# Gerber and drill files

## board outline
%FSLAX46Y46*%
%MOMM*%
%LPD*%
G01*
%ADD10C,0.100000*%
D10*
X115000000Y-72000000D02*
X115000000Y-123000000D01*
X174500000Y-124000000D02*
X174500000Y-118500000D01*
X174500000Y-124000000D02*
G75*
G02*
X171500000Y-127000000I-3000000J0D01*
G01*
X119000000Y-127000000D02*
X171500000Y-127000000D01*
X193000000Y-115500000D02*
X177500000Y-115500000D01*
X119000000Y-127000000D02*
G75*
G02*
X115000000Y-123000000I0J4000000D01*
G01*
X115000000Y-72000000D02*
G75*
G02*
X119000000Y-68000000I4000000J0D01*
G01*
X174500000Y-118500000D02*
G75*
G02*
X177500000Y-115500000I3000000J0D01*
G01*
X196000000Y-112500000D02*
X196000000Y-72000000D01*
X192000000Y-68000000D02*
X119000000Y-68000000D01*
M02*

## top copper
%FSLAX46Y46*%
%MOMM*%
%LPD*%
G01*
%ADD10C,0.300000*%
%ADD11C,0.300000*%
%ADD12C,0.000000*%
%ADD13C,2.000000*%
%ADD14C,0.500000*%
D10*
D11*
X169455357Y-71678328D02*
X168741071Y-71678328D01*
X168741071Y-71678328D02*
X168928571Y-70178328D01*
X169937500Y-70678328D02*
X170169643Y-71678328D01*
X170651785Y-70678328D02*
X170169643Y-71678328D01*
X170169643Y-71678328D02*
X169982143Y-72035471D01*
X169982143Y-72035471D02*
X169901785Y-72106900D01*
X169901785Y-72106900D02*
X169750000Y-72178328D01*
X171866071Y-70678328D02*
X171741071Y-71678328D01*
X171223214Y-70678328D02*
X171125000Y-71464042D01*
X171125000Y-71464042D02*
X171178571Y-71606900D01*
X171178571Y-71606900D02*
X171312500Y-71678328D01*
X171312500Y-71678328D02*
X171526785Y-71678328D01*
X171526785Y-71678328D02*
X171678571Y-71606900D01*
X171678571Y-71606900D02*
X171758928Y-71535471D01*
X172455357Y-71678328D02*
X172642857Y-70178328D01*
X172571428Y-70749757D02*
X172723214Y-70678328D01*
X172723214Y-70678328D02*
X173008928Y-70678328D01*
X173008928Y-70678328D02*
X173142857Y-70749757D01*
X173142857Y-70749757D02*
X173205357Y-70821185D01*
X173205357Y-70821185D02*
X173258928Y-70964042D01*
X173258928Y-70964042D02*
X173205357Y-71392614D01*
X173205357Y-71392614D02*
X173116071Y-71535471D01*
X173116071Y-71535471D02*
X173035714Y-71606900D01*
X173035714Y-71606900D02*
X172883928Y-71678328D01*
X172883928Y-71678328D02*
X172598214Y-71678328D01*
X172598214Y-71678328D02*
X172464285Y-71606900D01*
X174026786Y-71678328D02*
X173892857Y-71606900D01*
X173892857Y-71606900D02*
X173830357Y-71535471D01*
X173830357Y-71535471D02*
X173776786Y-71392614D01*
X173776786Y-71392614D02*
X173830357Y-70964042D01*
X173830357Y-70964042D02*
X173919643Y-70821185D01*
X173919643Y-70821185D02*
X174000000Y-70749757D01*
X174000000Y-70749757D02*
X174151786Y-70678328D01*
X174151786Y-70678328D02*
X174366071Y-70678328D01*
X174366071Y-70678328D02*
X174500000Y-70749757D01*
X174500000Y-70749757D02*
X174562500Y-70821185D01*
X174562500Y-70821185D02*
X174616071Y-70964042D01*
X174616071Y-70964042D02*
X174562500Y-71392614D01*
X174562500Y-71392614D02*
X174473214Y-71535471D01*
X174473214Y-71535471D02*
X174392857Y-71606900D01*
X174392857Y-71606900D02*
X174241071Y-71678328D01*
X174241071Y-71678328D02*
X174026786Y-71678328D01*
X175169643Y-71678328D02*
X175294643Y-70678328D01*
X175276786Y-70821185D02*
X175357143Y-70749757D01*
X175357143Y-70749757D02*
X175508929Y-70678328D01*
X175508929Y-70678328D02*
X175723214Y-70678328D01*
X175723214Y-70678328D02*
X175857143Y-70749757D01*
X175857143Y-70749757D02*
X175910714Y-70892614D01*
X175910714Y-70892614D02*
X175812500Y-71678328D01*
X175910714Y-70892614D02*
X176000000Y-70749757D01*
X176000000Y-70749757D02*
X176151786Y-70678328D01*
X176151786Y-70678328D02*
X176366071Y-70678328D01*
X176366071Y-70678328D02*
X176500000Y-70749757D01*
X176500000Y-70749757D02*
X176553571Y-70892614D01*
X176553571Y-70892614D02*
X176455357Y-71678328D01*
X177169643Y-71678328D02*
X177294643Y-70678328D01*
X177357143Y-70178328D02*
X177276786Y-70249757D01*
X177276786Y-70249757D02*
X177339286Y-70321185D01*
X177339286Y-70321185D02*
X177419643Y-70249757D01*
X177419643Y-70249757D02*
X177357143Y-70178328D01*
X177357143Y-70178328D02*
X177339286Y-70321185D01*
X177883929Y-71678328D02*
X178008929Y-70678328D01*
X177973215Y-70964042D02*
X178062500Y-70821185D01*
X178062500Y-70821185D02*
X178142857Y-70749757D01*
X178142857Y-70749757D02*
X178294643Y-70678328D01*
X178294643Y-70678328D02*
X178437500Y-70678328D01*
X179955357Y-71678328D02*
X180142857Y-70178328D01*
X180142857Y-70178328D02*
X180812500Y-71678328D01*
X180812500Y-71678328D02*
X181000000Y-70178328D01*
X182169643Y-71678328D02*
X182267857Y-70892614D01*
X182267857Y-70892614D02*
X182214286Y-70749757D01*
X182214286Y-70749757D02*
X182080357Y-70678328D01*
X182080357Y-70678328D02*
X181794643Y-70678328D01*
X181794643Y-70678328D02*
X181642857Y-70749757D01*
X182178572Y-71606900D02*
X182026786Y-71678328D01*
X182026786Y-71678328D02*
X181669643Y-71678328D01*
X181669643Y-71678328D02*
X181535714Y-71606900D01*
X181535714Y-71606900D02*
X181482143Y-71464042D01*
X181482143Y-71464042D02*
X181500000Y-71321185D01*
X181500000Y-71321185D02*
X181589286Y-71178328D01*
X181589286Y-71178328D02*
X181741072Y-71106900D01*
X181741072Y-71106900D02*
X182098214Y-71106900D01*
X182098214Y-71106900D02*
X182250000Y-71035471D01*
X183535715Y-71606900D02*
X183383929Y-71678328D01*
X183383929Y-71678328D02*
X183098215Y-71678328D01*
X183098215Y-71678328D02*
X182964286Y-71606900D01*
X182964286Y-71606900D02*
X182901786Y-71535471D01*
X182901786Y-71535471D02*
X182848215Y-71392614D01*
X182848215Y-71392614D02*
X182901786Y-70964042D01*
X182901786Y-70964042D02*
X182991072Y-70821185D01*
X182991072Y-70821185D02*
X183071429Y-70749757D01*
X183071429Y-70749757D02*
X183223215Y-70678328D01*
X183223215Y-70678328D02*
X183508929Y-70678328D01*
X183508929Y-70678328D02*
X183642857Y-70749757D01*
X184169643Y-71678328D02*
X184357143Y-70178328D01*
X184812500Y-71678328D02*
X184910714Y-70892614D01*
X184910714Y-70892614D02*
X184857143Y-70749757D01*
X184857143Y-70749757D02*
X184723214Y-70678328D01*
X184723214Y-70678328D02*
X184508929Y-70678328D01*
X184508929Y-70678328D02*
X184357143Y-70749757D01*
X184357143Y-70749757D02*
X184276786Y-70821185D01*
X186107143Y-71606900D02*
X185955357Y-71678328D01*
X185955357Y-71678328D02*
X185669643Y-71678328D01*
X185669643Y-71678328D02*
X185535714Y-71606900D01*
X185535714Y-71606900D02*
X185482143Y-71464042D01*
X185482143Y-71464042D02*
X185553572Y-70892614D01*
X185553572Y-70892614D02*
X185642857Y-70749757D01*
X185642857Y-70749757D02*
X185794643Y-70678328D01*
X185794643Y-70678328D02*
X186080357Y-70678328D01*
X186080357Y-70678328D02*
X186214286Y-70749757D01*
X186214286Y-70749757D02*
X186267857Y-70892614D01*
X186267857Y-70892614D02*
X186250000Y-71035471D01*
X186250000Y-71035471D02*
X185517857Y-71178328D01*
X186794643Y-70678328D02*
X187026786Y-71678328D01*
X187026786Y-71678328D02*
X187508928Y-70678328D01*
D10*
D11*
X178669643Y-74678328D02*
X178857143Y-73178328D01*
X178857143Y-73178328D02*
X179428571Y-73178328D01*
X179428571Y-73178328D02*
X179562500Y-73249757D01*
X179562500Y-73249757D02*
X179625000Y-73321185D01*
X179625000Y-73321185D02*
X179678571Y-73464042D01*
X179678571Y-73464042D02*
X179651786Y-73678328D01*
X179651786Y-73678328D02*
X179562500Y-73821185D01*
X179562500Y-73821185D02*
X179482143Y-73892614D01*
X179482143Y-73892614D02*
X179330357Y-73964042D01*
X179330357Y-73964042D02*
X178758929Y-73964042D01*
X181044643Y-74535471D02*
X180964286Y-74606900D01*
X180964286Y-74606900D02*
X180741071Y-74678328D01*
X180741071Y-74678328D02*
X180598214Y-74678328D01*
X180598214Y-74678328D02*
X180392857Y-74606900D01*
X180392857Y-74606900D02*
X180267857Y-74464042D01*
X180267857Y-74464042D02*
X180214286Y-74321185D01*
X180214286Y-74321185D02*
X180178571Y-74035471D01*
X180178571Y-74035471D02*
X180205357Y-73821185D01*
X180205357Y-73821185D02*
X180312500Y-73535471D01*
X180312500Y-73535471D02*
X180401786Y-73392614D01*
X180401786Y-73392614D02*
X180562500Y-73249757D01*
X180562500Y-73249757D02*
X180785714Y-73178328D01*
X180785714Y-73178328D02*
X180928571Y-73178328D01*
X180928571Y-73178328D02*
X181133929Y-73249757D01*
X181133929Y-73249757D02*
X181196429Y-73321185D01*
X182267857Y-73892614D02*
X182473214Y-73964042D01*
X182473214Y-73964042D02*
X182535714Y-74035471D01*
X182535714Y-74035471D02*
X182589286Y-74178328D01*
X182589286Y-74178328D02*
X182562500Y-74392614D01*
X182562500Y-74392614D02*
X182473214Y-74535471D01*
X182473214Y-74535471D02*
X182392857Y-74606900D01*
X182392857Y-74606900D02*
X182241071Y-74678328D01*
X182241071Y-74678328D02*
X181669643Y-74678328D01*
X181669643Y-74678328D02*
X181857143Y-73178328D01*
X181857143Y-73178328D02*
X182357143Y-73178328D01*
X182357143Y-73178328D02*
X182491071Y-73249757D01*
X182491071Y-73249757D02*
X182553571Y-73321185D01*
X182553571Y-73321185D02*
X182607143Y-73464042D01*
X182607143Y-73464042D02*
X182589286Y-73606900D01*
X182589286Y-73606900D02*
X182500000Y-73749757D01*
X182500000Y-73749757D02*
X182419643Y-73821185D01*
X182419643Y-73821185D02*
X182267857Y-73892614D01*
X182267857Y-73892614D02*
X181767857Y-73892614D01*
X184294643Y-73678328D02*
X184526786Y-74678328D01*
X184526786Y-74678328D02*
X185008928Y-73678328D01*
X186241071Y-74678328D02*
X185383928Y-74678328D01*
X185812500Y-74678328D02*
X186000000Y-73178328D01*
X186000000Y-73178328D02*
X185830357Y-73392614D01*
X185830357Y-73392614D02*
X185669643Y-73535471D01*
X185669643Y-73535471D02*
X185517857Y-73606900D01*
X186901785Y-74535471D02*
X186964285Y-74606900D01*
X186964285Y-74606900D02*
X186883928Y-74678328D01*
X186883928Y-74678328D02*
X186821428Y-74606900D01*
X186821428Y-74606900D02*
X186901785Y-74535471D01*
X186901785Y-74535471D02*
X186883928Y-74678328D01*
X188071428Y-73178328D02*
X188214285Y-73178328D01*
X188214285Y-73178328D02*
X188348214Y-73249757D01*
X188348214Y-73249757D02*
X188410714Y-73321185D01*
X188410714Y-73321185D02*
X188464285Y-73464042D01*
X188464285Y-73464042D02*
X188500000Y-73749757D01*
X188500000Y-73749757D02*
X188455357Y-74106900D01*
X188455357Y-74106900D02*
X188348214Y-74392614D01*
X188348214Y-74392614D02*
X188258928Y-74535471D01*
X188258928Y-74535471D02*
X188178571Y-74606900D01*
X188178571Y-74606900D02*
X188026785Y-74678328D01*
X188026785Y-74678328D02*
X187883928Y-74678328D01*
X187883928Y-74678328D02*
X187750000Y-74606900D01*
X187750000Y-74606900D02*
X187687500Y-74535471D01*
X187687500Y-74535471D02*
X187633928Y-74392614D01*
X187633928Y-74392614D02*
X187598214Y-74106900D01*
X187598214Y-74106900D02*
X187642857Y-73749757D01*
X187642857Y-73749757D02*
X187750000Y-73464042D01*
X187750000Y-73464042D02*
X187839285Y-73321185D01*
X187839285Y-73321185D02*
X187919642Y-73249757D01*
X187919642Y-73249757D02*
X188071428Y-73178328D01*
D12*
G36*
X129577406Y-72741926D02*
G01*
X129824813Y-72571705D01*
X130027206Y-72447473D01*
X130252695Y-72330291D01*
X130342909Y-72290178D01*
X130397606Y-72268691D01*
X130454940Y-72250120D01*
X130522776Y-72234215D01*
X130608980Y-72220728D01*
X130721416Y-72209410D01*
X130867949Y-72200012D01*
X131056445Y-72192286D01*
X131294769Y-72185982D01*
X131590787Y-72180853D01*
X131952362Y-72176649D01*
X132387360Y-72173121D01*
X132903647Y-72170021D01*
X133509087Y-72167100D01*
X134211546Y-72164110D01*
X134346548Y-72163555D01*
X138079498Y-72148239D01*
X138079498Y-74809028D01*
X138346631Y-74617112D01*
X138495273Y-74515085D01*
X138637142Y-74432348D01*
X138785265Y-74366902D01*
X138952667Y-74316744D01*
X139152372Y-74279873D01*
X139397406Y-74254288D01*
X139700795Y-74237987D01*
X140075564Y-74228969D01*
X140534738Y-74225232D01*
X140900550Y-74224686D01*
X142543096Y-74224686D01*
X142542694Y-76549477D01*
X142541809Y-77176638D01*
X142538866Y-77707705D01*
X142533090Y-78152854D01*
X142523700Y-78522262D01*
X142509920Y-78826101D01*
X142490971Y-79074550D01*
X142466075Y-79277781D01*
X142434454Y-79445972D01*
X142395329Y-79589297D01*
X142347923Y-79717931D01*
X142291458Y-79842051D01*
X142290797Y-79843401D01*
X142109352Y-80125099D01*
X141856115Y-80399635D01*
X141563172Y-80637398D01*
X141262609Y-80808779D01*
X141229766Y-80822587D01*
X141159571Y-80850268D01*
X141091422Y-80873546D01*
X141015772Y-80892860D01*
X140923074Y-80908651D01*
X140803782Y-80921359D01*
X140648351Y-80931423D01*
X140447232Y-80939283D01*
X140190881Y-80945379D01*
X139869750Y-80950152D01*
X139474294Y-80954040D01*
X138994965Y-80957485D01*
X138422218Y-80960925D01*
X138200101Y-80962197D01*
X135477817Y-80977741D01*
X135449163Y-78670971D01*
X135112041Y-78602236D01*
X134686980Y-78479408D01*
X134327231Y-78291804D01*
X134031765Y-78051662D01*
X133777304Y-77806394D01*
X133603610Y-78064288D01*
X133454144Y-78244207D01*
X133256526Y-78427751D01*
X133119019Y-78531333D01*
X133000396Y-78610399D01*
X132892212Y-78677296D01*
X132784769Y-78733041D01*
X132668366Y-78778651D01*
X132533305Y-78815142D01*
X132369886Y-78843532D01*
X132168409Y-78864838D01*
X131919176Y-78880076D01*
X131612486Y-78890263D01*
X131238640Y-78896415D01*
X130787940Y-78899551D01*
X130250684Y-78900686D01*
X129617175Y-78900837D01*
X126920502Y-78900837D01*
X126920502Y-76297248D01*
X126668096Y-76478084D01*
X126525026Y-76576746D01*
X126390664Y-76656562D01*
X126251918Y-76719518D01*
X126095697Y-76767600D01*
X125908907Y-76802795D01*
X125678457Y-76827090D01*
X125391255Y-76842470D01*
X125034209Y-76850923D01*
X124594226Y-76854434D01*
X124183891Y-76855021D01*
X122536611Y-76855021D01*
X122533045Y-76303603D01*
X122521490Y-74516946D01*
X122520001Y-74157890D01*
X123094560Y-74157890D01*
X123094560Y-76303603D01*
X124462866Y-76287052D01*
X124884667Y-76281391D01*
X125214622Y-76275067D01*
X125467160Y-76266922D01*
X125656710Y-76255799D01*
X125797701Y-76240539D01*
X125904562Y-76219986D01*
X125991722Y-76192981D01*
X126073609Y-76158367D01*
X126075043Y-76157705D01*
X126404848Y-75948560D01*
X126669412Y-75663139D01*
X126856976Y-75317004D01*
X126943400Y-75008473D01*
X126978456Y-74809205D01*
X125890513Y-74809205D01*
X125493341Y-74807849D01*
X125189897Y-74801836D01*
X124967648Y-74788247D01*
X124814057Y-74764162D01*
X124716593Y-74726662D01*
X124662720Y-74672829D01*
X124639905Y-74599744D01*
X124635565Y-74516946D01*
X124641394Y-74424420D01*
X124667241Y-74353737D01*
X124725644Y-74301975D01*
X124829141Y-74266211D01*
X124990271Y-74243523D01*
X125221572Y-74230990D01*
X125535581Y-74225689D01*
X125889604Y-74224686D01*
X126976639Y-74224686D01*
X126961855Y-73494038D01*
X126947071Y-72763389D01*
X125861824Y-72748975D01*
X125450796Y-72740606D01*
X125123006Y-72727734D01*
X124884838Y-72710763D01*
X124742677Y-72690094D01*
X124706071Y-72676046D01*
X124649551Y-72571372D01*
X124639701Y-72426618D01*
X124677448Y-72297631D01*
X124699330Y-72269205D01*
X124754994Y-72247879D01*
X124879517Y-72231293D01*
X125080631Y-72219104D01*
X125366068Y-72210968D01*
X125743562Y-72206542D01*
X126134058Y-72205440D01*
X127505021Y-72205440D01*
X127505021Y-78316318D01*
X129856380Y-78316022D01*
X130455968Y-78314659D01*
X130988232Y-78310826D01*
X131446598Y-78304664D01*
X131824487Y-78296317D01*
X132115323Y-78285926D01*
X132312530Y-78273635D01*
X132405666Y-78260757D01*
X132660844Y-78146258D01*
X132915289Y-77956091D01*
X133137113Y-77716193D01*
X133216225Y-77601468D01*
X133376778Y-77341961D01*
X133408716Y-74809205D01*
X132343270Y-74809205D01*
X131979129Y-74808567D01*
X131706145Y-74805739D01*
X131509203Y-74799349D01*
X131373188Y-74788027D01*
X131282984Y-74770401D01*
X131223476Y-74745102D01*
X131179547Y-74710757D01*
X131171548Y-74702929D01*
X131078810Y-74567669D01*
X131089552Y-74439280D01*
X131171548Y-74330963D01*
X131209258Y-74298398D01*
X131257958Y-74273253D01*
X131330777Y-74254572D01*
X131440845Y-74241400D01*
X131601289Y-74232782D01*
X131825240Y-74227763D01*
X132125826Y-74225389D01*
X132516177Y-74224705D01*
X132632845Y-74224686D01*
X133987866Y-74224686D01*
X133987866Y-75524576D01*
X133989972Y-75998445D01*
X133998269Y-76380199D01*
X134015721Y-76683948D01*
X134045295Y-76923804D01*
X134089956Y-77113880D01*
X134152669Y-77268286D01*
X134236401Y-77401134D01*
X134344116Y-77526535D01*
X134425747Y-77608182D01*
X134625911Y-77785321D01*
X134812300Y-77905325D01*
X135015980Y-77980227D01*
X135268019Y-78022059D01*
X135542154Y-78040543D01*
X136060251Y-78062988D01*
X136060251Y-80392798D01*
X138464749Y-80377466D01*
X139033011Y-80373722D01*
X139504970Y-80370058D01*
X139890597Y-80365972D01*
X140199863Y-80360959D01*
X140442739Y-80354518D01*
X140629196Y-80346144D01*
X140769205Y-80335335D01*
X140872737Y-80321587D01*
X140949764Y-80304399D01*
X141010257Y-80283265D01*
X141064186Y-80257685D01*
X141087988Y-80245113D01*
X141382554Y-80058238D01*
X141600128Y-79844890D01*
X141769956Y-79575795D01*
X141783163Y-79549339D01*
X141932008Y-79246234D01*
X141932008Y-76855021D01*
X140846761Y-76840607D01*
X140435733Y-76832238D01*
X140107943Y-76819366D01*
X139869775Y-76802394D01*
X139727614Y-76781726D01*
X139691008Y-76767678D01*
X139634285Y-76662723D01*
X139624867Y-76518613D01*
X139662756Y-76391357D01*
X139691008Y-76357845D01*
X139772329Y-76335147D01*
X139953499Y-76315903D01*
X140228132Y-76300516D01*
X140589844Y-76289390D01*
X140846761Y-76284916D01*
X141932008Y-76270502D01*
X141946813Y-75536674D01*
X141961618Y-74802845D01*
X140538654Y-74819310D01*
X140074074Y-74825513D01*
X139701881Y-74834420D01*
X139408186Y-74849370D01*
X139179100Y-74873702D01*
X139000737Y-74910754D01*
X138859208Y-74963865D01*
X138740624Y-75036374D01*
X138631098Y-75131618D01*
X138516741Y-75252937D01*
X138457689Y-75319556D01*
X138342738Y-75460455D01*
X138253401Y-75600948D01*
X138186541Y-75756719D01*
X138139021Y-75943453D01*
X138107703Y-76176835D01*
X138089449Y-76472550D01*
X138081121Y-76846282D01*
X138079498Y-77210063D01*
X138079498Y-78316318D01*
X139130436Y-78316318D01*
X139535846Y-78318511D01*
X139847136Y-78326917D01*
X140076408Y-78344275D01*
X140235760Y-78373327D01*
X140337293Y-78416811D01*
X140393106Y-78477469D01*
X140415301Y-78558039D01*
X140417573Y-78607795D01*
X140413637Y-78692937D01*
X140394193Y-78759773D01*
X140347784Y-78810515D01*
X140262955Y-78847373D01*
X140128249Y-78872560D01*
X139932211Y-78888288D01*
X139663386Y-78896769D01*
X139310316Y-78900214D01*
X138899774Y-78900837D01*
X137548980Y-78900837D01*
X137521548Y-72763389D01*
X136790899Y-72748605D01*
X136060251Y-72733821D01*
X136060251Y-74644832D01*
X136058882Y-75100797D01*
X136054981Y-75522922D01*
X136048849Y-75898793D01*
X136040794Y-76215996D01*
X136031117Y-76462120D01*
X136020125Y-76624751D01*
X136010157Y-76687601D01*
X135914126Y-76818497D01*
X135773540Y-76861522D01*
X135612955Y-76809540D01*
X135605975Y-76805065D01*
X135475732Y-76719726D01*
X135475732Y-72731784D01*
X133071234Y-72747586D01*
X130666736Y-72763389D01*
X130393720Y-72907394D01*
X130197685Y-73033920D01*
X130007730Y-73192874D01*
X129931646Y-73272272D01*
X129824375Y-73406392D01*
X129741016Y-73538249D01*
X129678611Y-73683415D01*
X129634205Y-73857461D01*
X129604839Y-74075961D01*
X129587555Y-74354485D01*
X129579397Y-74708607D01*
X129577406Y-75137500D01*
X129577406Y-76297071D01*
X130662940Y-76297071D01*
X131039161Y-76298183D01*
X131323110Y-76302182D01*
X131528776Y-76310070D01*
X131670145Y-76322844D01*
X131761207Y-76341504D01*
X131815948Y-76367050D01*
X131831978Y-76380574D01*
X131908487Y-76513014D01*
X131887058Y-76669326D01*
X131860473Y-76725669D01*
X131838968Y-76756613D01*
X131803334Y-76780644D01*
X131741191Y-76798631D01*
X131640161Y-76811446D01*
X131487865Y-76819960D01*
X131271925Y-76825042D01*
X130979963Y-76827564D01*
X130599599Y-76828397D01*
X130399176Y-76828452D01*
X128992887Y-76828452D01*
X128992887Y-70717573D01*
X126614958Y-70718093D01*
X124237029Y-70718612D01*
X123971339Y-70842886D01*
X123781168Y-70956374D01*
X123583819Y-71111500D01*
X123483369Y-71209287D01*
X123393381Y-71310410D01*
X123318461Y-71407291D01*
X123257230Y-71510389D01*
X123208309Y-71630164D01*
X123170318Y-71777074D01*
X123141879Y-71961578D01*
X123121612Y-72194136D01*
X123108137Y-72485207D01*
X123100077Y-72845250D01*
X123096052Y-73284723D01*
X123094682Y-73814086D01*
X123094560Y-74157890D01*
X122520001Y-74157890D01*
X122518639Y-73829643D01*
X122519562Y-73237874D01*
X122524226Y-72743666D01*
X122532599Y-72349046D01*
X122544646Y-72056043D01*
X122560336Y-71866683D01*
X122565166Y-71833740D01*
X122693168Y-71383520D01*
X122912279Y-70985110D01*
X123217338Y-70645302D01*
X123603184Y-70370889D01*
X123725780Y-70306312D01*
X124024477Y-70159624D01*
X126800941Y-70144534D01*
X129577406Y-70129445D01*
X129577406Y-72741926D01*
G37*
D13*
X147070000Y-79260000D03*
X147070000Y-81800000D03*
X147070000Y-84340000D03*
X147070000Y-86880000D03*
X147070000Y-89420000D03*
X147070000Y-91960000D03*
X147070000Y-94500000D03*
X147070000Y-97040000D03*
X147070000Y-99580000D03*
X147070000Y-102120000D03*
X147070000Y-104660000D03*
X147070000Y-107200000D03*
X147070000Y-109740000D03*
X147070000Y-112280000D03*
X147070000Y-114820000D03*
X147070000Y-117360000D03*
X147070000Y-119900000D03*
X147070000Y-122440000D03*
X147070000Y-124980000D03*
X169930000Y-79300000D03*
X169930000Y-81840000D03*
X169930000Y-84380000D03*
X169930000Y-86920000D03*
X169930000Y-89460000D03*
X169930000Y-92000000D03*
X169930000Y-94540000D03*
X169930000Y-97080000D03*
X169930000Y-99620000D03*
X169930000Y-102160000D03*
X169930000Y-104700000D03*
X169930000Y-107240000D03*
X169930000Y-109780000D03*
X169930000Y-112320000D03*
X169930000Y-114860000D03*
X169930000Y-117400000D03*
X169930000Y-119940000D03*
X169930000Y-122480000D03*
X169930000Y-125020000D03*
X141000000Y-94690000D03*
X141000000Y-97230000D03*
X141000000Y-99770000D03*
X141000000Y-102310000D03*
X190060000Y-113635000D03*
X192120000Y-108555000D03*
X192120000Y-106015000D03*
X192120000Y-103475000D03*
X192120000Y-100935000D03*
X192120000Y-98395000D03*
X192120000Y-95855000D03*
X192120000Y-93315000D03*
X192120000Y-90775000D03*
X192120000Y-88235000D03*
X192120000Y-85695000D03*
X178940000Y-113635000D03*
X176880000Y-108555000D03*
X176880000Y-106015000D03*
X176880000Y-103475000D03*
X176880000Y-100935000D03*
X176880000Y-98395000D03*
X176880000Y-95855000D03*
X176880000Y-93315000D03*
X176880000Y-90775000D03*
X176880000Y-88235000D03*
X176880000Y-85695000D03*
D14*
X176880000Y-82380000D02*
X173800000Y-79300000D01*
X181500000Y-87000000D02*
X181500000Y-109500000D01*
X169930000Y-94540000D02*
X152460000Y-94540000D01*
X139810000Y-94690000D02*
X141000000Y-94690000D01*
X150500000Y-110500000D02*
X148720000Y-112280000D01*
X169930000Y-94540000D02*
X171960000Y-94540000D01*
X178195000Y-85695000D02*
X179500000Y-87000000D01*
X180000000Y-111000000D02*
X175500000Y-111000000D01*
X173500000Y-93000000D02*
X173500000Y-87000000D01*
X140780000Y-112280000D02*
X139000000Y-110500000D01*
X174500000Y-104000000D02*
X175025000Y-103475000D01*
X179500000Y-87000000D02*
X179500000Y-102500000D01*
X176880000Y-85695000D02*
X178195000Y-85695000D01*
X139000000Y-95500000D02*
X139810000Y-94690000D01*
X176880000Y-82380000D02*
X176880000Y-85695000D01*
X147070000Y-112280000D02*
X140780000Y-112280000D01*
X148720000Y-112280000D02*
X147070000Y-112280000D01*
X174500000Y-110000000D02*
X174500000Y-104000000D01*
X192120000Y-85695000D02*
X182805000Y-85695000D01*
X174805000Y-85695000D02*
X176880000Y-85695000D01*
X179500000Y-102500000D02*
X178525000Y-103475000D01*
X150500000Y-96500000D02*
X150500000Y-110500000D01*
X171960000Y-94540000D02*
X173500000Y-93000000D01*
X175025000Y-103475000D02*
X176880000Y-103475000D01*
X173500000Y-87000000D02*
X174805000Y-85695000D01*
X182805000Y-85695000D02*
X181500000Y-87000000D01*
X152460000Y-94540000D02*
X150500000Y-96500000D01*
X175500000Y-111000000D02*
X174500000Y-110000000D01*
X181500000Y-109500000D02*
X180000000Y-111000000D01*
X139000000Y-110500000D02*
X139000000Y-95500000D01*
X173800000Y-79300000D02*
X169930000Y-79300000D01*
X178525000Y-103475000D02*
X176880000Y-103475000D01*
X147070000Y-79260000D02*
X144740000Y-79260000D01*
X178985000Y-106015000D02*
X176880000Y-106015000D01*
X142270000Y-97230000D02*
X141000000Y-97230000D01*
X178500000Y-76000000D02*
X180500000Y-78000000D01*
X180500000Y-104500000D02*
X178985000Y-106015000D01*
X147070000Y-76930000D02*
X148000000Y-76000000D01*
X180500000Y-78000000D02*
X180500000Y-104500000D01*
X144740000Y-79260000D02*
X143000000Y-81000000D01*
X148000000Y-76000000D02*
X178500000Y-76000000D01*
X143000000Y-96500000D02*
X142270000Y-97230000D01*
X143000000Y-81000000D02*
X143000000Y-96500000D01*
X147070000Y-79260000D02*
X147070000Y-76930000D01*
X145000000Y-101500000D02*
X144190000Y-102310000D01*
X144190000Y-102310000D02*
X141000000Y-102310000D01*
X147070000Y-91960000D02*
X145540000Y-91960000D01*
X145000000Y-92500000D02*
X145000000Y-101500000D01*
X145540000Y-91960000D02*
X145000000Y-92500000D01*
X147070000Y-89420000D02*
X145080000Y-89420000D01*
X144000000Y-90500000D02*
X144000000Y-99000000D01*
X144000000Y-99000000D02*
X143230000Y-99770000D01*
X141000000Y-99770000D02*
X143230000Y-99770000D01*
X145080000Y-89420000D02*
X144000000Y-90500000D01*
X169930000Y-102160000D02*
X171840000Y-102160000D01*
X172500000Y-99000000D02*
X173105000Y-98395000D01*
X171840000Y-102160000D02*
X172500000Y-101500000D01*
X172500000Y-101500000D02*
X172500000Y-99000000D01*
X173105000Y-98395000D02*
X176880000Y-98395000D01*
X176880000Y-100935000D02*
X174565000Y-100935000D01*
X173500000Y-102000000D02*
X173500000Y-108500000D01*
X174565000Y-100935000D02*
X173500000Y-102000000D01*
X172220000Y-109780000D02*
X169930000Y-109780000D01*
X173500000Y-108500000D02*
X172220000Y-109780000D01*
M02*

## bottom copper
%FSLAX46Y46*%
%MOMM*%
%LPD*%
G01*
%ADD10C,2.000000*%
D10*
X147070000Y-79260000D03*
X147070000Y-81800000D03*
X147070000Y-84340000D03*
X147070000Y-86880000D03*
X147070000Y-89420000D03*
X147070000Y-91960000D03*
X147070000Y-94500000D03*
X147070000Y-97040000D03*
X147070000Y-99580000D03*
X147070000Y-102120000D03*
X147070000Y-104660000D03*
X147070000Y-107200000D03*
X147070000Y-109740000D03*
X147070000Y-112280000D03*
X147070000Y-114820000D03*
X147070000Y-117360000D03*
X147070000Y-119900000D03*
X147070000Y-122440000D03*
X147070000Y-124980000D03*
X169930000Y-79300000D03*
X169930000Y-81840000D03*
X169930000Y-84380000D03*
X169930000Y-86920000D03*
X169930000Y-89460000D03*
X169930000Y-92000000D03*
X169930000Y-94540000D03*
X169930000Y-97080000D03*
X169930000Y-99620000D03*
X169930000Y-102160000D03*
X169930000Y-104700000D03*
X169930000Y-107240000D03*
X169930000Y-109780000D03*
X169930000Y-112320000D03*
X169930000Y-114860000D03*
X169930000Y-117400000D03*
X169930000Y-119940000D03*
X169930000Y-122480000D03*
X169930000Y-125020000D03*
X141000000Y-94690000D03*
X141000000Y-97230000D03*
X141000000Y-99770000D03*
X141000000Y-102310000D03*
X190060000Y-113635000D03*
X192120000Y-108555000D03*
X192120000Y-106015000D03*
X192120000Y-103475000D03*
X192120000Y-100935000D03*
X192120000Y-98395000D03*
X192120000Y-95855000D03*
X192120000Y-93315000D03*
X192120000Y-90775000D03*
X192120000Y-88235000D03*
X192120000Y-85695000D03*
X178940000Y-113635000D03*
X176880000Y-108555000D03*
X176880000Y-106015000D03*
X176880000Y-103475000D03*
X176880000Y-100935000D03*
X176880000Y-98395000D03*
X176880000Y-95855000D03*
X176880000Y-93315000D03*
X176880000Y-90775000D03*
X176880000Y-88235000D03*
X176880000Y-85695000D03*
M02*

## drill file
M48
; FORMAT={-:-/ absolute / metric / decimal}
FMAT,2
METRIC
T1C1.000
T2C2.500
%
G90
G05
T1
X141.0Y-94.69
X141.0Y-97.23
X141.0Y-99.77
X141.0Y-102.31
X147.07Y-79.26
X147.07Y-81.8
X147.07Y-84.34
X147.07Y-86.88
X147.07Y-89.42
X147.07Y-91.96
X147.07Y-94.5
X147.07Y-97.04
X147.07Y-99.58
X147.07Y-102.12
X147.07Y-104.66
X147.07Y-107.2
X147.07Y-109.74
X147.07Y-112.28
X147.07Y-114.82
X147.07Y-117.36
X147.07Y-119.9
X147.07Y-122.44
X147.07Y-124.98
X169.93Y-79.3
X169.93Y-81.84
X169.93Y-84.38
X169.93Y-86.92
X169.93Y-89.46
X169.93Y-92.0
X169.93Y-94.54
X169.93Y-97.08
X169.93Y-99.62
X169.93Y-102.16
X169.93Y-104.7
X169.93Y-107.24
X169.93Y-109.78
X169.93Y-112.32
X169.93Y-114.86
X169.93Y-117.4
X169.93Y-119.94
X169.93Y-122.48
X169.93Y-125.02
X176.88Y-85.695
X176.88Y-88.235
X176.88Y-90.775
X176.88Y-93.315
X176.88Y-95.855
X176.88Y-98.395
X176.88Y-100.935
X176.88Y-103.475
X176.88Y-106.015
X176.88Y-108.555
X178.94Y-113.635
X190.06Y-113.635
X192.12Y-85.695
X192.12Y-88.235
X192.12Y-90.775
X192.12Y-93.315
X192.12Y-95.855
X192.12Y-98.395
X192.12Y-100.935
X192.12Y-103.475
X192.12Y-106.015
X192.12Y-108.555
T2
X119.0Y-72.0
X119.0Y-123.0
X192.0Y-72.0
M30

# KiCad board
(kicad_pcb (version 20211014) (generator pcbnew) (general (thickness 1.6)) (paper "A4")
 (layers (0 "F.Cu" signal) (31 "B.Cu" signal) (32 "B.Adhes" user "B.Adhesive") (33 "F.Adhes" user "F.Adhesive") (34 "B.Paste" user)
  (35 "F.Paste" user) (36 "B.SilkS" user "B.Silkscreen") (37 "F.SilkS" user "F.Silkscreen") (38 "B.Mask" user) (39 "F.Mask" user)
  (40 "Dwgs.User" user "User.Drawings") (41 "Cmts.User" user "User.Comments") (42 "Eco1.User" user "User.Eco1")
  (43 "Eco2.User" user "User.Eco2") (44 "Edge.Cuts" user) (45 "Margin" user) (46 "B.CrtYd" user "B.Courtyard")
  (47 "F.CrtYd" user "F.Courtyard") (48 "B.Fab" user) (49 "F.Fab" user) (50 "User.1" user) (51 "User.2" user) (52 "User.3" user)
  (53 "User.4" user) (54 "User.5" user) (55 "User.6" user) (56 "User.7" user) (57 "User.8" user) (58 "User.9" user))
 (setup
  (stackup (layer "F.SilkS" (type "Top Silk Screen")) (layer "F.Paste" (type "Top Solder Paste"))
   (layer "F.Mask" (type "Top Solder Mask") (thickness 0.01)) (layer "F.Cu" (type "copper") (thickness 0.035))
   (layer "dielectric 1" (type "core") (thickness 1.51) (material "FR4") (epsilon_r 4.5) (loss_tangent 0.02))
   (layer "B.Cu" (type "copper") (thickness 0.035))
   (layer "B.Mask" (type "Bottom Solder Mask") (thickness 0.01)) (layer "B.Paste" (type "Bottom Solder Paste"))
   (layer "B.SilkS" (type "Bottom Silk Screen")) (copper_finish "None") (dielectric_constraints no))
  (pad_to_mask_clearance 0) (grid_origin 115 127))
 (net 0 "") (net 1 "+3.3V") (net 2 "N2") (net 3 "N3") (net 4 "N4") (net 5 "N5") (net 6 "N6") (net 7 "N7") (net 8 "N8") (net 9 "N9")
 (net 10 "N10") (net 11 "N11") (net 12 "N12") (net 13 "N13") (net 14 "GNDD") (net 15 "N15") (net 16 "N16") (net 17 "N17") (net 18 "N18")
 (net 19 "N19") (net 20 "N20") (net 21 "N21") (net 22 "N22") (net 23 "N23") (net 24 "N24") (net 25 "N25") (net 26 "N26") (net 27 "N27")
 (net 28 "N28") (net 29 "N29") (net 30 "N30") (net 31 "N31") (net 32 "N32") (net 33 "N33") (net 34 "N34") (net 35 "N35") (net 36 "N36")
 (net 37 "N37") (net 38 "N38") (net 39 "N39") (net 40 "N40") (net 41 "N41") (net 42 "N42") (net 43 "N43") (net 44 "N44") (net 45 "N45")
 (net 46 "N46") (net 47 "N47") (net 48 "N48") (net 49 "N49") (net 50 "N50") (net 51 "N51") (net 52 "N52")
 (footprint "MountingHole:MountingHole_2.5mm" (layer "F.Cu") (at 119 123 180)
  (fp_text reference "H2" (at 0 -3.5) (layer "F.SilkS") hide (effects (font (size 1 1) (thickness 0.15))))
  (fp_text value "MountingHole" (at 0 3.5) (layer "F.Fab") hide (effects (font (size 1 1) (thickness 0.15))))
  (pad "" np_thru_hole circle (at 0 0 180) (size 2.5 2.5) (drill 2.5) (layers *.Cu *.Mask)))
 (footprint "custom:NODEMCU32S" (layer "F.Cu") (at 158.5 104.5)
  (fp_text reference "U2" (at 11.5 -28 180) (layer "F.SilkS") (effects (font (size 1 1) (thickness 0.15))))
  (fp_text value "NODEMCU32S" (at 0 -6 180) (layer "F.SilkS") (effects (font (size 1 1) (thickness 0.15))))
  (pad "1" thru_hole circle (at -11.43 -25.24) (size 2 2) (drill 1) (layers *.Cu *.Mask) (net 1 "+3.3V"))
  (pad "2" thru_hole circle (at -11.43 -22.7) (size 2 2) (drill 1) (layers *.Cu *.Mask) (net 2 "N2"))
  (pad "3" thru_hole circle (at -11.43 -20.16) (size 2 2) (drill 1) (layers *.Cu *.Mask) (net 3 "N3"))
  (pad "4" thru_hole circle (at -11.43 -17.62) (size 2 2) (drill 1) (layers *.Cu *.Mask) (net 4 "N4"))
  (pad "5" thru_hole circle (at -11.43 -15.08) (size 2 2) (drill 1) (layers *.Cu *.Mask) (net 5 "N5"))
  (pad "6" thru_hole circle (at -11.43 -12.54) (size 2 2) (drill 1) (layers *.Cu *.Mask) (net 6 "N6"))
  (pad "7" thru_hole circle (at -11.43 -10) (size 2 2) (drill 1) (layers *.Cu *.Mask) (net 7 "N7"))
  (pad "8" thru_hole circle (at -11.43 -7.46) (size 2 2) (drill 1) (layers *.Cu *.Mask) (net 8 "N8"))
  (pad "9" thru_hole circle (at -11.43 -4.92) (size 2 2) (drill 1) (layers *.Cu *.Mask) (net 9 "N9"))
  (pad "10" thru_hole circle (at -11.43 -2.38) (size 2 2) (drill 1) (layers *.Cu *.Mask) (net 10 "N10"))
  (pad "11" thru_hole circle (at -11.43 0.16) (size 2 2) (drill 1) (layers *.Cu *.Mask) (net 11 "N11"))
  (pad "12" thru_hole circle (at -11.43 2.7) (size 2 2) (drill 1) (layers *.Cu *.Mask) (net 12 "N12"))
  (pad "13" thru_hole circle (at -11.43 5.24) (size 2 2) (drill 1) (layers *.Cu *.Mask) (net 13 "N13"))
  (pad "14" thru_hole circle (at -11.43 7.78) (size 2 2) (drill 1) (layers *.Cu *.Mask) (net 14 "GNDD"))
  (pad "15" thru_hole circle (at -11.43 10.32) (size 2 2) (drill 1) (layers *.Cu *.Mask) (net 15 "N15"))
  (pad "16" thru_hole circle (at -11.43 12.86) (size 2 2) (drill 1) (layers *.Cu *.Mask) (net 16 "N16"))
  (pad "17" thru_hole circle (at -11.43 15.4) (size 2 2) (drill 1) (layers *.Cu *.Mask) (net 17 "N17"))
  (pad "18" thru_hole circle (at -11.43 17.94) (size 2 2) (drill 1) (layers *.Cu *.Mask) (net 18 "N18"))
  (pad "19" thru_hole circle (at -11.43 20.48) (size 2 2) (drill 1) (layers *.Cu *.Mask) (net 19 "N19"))
  (pad "20" thru_hole circle (at 11.43 -25.2) (size 2 2) (drill 1) (layers *.Cu *.Mask) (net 14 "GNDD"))
  (pad "21" thru_hole circle (at 11.43 -22.66) (size 2 2) (drill 1) (layers *.Cu *.Mask) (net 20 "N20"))
  (pad "22" thru_hole circle (at 11.43 -20.12) (size 2 2) (drill 1) (layers *.Cu *.Mask) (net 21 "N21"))
  (pad "23" thru_hole circle (at 11.43 -17.58) (size 2 2) (drill 1) (layers *.Cu *.Mask) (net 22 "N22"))
  (pad "24" thru_hole circle (at 11.43 -15.04) (size 2 2) (drill 1) (layers *.Cu *.Mask) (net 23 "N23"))
  (pad "25" thru_hole circle (at 11.43 -12.5) (size 2 2) (drill 1) (layers *.Cu *.Mask) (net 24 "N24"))
  (pad "26" thru_hole circle (at 11.43 -9.96) (size 2 2) (drill 1) (layers *.Cu *.Mask) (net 14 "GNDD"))
  (pad "27" thru_hole circle (at 11.43 -7.42) (size 2 2) (drill 1) (layers *.Cu *.Mask) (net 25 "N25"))
  (pad "28" thru_hole circle (at 11.43 -4.88) (size 2 2) (drill 1) (layers *.Cu *.Mask) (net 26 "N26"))
  (pad "29" thru_hole circle (at 11.43 -2.34) (size 2 2) (drill 1) (layers *.Cu *.Mask) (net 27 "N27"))
  (pad "30" thru_hole circle (at 11.43 0.2) (size 2 2) (drill 1) (layers *.Cu *.Mask) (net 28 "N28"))
  (pad "31" thru_hole circle (at 11.43 2.74) (size 2 2) (drill 1) (layers *.Cu *.Mask) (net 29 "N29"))
  (pad "32" thru_hole circle (at 11.43 5.28) (size 2 2) (drill 1) (layers *.Cu *.Mask) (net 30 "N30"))
  (pad "33" thru_hole circle (at 11.43 7.82) (size 2 2) (drill 1) (layers *.Cu *.Mask) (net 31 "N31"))
  (pad "34" thru_hole circle (at 11.43 10.36) (size 2 2) (drill 1) (layers *.Cu *.Mask) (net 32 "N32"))
  (pad "35" thru_hole circle (at 11.43 12.9) (size 2 2) (drill 1) (layers *.Cu *.Mask) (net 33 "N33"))
  (pad "36" thru_hole circle (at 11.43 15.44) (size 2 2) (drill 1) (layers *.Cu *.Mask) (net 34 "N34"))
  (pad "37" thru_hole circle (at 11.43 17.98) (size 2 2) (drill 1) (layers *.Cu *.Mask) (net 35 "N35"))
  (pad "38" thru_hole circle (at 11.43 20.52) (size 2 2) (drill 1) (layers *.Cu *.Mask) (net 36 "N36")))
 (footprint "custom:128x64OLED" (layer "F.Cu") (at 129 98.5 -90)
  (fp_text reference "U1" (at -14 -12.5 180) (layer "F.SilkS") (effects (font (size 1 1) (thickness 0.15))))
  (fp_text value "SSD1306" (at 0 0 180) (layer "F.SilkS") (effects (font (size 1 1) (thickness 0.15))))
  (pad "1" thru_hole circle (at -3.81 -12) (size 2 2) (drill 1) (layers *.Cu *.Mask) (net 14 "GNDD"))
  (pad "2" thru_hole circle (at -1.27 -12) (size 2 2) (drill 1) (layers *.Cu *.Mask) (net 1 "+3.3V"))
  (pad "3" thru_hole circle (at 1.27 -12) (size 2 2) (drill 1) (layers *.Cu *.Mask) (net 5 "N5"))
  (pad "4" thru_hole circle (at 3.81 -12) (size 2 2) (drill 1) (layers *.Cu *.Mask) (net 6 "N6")))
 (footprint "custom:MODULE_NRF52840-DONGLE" (layer "F.Cu") (at 184.5 103 -90)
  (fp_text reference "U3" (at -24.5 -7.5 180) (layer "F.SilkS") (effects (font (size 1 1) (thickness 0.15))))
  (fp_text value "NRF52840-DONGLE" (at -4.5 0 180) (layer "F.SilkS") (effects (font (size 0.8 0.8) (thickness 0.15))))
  (pad "1" thru_hole circle (at 10.635 -5.56 270) (size 2 2) (drill 1) (layers *.Cu *.Mask) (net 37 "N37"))
  (pad "2" thru_hole circle (at 5.555 -7.62 270) (size 2 2) (drill 1) (layers *.Cu *.Mask) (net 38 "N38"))
  (pad "3" thru_hole circle (at 3.015 -7.62 270) (size 2 2) (drill 1) (layers *.Cu *.Mask) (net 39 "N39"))
  (pad "4" thru_hole circle (at 0.475 -7.62 270) (size 2 2) (drill 1) (layers *.Cu *.Mask) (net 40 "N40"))
  (pad "5" thru_hole circle (at -2.065 -7.62 270) (size 2 2) (drill 1) (layers *.Cu *.Mask) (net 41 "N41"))
  (pad "6" thru_hole circle (at -4.605 -7.62 270) (size 2 2) (drill 1) (layers *.Cu *.Mask) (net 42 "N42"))
  (pad "7" thru_hole circle (at -7.145 -7.62 270) (size 2 2) (drill 1) (layers *.Cu *.Mask) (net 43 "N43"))
  (pad "8" thru_hole circle (at -9.685 -7.62 270) (size 2 2) (drill 1) (layers *.Cu *.Mask) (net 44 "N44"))
  (pad "9" thru_hole circle (at -12.225 -7.62 270) (size 2 2) (drill 1) (layers *.Cu *.Mask) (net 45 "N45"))
  (pad "10" thru_hole circle (at -14.765 -7.62 270) (size 2 2) (drill 1) (layers *.Cu *.Mask) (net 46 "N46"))
  (pad "11" thru_hole circle (at -17.305 -7.62 270) (size 2 2) (drill 1) (layers *.Cu *.Mask) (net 14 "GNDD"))
  (pad "12" thru_hole circle (at 10.635 5.56 270) (size 2 2) (drill 1) (layers *.Cu *.Mask) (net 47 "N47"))
  (pad "13" thru_hole circle (at 5.555 7.62 270) (size 2 2) (drill 1) (layers *.Cu *.Mask) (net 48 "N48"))
  (pad "14" thru_hole circle (at 3.015 7.62 270) (size 2 2) (drill 1) (layers *.Cu *.Mask) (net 1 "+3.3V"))
  (pad "15" thru_hole circle (at 0.475 7.62 270) (size 2 2) (drill 1) (layers *.Cu *.Mask) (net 14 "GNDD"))
  (pad "16" thru_hole circle (at -2.065 7.62 270) (size 2 2) (drill 1) (layers *.Cu *.Mask) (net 30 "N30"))
  (pad "17" thru_hole circle (at -4.605 7.62 270) (size 2 2) (drill 1) (layers *.Cu *.Mask) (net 27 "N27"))
  (pad "18" thru_hole circle (at -7.145 7.62 270) (size 2 2) (drill 1) (layers *.Cu *.Mask) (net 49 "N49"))
  (pad "19" thru_hole circle (at -9.685 7.62 270) (size 2 2) (drill 1) (layers *.Cu *.Mask) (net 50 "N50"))
  (pad "20" thru_hole circle (at -12.225 7.62 270) (size 2 2) (drill 1) (layers *.Cu *.Mask) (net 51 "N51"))
  (pad "21" thru_hole circle (at -14.765 7.62 270) (size 2 2) (drill 1) (layers *.Cu *.Mask) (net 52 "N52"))
  (pad "22" thru_hole circle (at -17.305 7.62 270) (size 2 2) (drill 1) (layers *.Cu *.Mask) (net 14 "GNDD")))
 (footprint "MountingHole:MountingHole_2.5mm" (layer "F.Cu") (at 119 72)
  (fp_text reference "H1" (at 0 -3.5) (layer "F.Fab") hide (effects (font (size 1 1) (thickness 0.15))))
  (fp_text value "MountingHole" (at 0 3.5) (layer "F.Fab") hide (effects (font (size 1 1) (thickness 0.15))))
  (pad "" np_thru_hole circle (at 0 0) (size 2.5 2.5) (drill 2.5) (layers *.Cu *.Mask)))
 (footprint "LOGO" (layer "F.Cu") (at 132.5 75.5)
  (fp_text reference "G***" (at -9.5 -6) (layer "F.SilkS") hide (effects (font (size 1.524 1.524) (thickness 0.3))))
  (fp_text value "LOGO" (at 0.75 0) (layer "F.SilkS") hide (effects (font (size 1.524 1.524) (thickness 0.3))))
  (fp_poly
   (pts (xy -2.922594 -2.758074) (xy -2.675187 -2.928295) (xy -2.472794 -3.052527) (xy -2.247305 -3.169709) (xy -2.157091 -3.209822)
    (xy -2.102394 -3.231309) (xy -2.04506 -3.24988) (xy -1.977224 -3.265785) (xy -1.89102 -3.279272) (xy -1.778584 -3.29059)
    (xy -1.632051 -3.299988) (xy -1.443555 -3.307714) (xy -1.205231 -3.314018) (xy -0.909213 -3.319147) (xy -0.547638 -3.323351)
    (xy -0.11264 -3.326879) (xy 0.403647 -3.329979) (xy 1.009087 -3.3329) (xy 1.711546 -3.33589) (xy 1.846548 -3.336445)
    (xy 5.579498 -3.351761) (xy 5.579498 -0.690972) (xy 5.846631 -0.882888) (xy 5.995273 -0.984915) (xy 6.137142 -1.067652)
    (xy 6.285265 -1.133098) (xy 6.452667 -1.183256) (xy 6.652372 -1.220127) (xy 6.897406 -1.245712) (xy 7.200795 -1.262013)
    (xy 7.575564 -1.271031) (xy 8.034738 -1.274768) (xy 8.40055 -1.275314) (xy 10.043096 -1.275314) (xy 10.042694 1.049477)
    (xy 10.041809 1.676638) (xy 10.038866 2.207705) (xy 10.03309 2.652854) (xy 10.0237 3.022262) (xy 10.00992 3.326101)
    (xy 9.990971 3.57455) (xy 9.966075 3.777781) (xy 9.934454 3.945972) (xy 9.895329 4.089297) (xy 9.847923 4.217931) (xy 9.791458 4.342051)
    (xy 9.790797 4.343401) (xy 9.609352 4.625099) (xy 9.356115 4.899635) (xy 9.063172 5.137398) (xy 8.762609 5.308779)
    (xy 8.729766 5.322587) (xy 8.659571 5.350268) (xy 8.591422 5.373546) (xy 8.515772 5.39286) (xy 8.423074 5.408651) (xy 8.303782 5.421359)
    (xy 8.148351 5.431423) (xy 7.947232 5.439283) (xy 7.690881 5.445379) (xy 7.36975 5.450152) (xy 6.974294 5.45404) (xy 6.494965 5.457485)
    (xy 5.922218 5.460925) (xy 5.700101 5.462197) (xy 2.977817 5.477741) (xy 2.949163 3.170971) (xy 2.612041 3.102236) (xy 2.18698 2.979408)
    (xy 1.827231 2.791804) (xy 1.531765 2.551662) (xy 1.277304 2.306394) (xy 1.10361 2.564288) (xy 0.954144 2.744207) (xy 0.756526 2.927751)
    (xy 0.619019 3.031333) (xy 0.500396 3.110399) (xy 0.392212 3.177296) (xy 0.284769 3.233041) (xy 0.168366 3.278651)
    (xy 0.033305 3.315142) (xy -0.130114 3.343532) (xy -0.331591 3.364838) (xy -0.580824 3.380076) (xy -0.887514 3.390263)
    (xy -1.26136 3.396415) (xy -1.71206 3.399551) (xy -2.249316 3.400686) (xy -2.882825 3.400837) (xy -5.579498 3.400837)
    (xy -5.579498 0.797248) (xy -5.831904 0.978084) (xy -5.974974 1.076746) (xy -6.109336 1.156562) (xy -6.248082 1.219518)
    (xy -6.404303 1.2676) (xy -6.591093 1.302795) (xy -6.821543 1.32709) (xy -7.108745 1.34247) (xy -7.465791 1.350923)
    (xy -7.905774 1.354434) (xy -8.316109 1.355021) (xy -9.963389 1.355021) (xy -9.966955 0.803603) (xy -9.40544 0.803603)
    (xy -8.037134 0.787052) (xy -7.615333 0.781391) (xy -7.285378 0.775067) (xy -7.03284 0.766922) (xy -6.84329 0.755799)
    (xy -6.702299 0.740539) (xy -6.595438 0.719986) (xy -6.508278 0.692981) (xy -6.426391 0.658367) (xy -6.424957 0.657705)
    (xy -6.095152 0.44856) (xy -5.830588 0.163139) (xy -5.643024 -0.182996) (xy -5.5566 -0.491527) (xy -5.521544 -0.690795)
    (xy -6.609487 -0.690795) (xy -7.006659 -0.692151) (xy -7.310103 -0.698164) (xy -7.532352 -0.711753) (xy -7.685943 -0.735838)
    (xy -7.783407 -0.773338) (xy -7.83728 -0.827171) (xy -7.860095 -0.900256) (xy -7.864435 -0.983054) (xy -7.858606 -1.07558)
    (xy -7.832759 -1.146263) (xy -7.774356 -1.198025) (xy -7.670859 -1.233789) (xy -7.509729 -1.256477) (xy -7.278428 -1.26901)
    (xy -6.964419 -1.274311) (xy -6.610396 -1.275314) (xy -5.523361 -1.275314) (xy -5.538145 -2.005962) (xy -5.552929 -2.736611)
    (xy -6.638176 -2.751025) (xy -7.049204 -2.759394) (xy -7.376994 -2.772266) (xy -7.615162 -2.789237) (xy -7.757323 -2.809906)
    (xy -7.793929 -2.823954) (xy -7.850449 -2.928628) (xy -7.860299 -3.073382) (xy -7.822552 -3.202369) (xy -7.80067 -3.230795)
    (xy -7.745006 -3.252121) (xy -7.620483 -3.268707) (xy -7.419369 -3.280896) (xy -7.133932 -3.289032) (xy -6.756438 -3.293458)
    (xy -6.365942 -3.29456) (xy -4.994979 -3.29456) (xy -4.994979 2.816318) (xy -2.64362 2.816022) (xy -2.044032 2.814659)
    (xy -1.511768 2.810826) (xy -1.053402 2.804664) (xy -0.675513 2.796317) (xy -0.384677 2.785926) (xy -0.18747 2.773635)
    (xy -0.094334 2.760757) (xy 0.160844 2.646258) (xy 0.415289 2.456091) (xy 0.637113 2.216193) (xy 0.716225 2.101468)
    (xy 0.876778 1.841961) (xy 0.908716 -0.690795) (xy -0.15673 -0.690795) (xy -0.520871 -0.691433) (xy -0.793855 -0.694261)
    (xy -0.990797 -0.700651) (xy -1.126812 -0.711973) (xy -1.217016 -0.729599) (xy -1.276524 -0.754898) (xy -1.320453 -0.789243)
    (xy -1.328452 -0.797071) (xy -1.42119 -0.932331) (xy -1.410448 -1.06072) (xy -1.328452 -1.169037) (xy -1.290742 -1.201602)
    (xy -1.242042 -1.226747) (xy -1.169223 -1.245428) (xy -1.059155 -1.2586) (xy -0.898711 -1.267218) (xy -0.67476 -1.272237)
    (xy -0.374174 -1.274611) (xy 0.016177 -1.275295) (xy 0.132845 -1.275314) (xy 1.487866 -1.275314) (xy 1.487866 0.024576)
    (xy 1.489972 0.498445) (xy 1.498269 0.880199) (xy 1.515721 1.183948) (xy 1.545295 1.423804) (xy 1.589956 1.61388) (xy 1.652669 1.768286)
    (xy 1.736401 1.901134) (xy 1.844116 2.026535) (xy 1.925747 2.108182) (xy 2.125911 2.285321) (xy 2.3123 2.405325) (xy 2.51598 2.480227)
    (xy 2.768019 2.522059) (xy 3.042154 2.540543) (xy 3.560251 2.562988) (xy 3.560251 4.892798) (xy 5.964749 4.877466)
    (xy 6.533011 4.873722) (xy 7.00497 4.870058) (xy 7.390597 4.865972) (xy 7.699863 4.860959) (xy 7.942739 4.854518) (xy 8.129196 4.846144)
    (xy 8.269205 4.835335) (xy 8.372737 4.821587) (xy 8.449764 4.804399) (xy 8.510257 4.783265) (xy 8.564186 4.757685)
    (xy 8.587988 4.745113) (xy 8.882554 4.558238) (xy 9.100128 4.34489) (xy 9.269956 4.075795) (xy 9.283163 4.049339) (xy 9.432008 3.746234)
    (xy 9.432008 1.355021) (xy 8.346761 1.340607) (xy 7.935733 1.332238) (xy 7.607943 1.319366) (xy 7.369775 1.302394)
    (xy 7.227614 1.281726) (xy 7.191008 1.267678) (xy 7.134285 1.162723) (xy 7.124867 1.018613) (xy 7.162756 0.891357)
    (xy 7.191008 0.857845) (xy 7.272329 0.835147) (xy 7.453499 0.815903) (xy 7.728132 0.800516) (xy 8.089844 0.78939) (xy 8.346761 0.784916)
    (xy 9.432008 0.770502) (xy 9.446813 0.036674) (xy 9.461618 -0.697155) (xy 8.038654 -0.68069) (xy 7.574074 -0.674487)
    (xy 7.201881 -0.66558) (xy 6.908186 -0.65063) (xy 6.6791 -0.626298) (xy 6.500737 -0.589246) (xy 6.359208 -0.536135)
    (xy 6.240624 -0.463626) (xy 6.131098 -0.368382) (xy 6.016741 -0.247063) (xy 5.957689 -0.180444) (xy 5.842738 -0.039545)
    (xy 5.753401 0.100948) (xy 5.686541 0.256719) (xy 5.639021 0.443453) (xy 5.607703 0.676835) (xy 5.589449 0.97255) (xy 5.581121 1.346282)
    (xy 5.579498 1.710063) (xy 5.579498 2.816318) (xy 6.630436 2.816318) (xy 7.035846 2.818511) (xy 7.347136 2.826917)
    (xy 7.576408 2.844275) (xy 7.73576 2.873327) (xy 7.837293 2.916811) (xy 7.893106 2.977469) (xy 7.915301 3.058039) (xy 7.917573 3.107795)
    (xy 7.913637 3.192937) (xy 7.894193 3.259773) (xy 7.847784 3.310515) (xy 7.762955 3.347373) (xy 7.628249 3.37256) (xy 7.432211 3.388288)
    (xy 7.163386 3.396769) (xy 6.810316 3.400214) (xy 6.399774 3.400837) (xy 5.04898 3.400837) (xy 5.021548 -2.736611)
    (xy 4.290899 -2.751395) (xy 3.560251 -2.766179) (xy 3.560251 -0.855168) (xy 3.558882 -0.399203) (xy 3.554981 0.022922)
    (xy 3.548849 0.398793) (xy 3.540794 0.715996) (xy 3.531117 0.96212) (xy 3.520125 1.124751) (xy 3.510157 1.187601) (xy 3.414126 1.318497)
    (xy 3.27354 1.361522) (xy 3.112955 1.30954) (xy 3.105975 1.305065) (xy 2.975732 1.219726) (xy 2.975732 -2.768216)
    (xy 0.571234 -2.752414) (xy -1.833264 -2.736611) (xy -2.10628 -2.592606) (xy -2.302315 -2.46608) (xy -2.49227 -2.307126)
    (xy -2.568354 -2.227728) (xy -2.675625 -2.093608) (xy -2.758984 -1.961751) (xy -2.821389 -1.816585) (xy -2.865795 -1.642539)
    (xy -2.895161 -1.424039) (xy -2.912445 -1.145515) (xy -2.920603 -0.791393) (xy -2.922594 -0.3625) (xy -2.922594 0.797071)
    (xy -1.83706 0.797071) (xy -1.460839 0.798183) (xy -1.17689 0.802182) (xy -0.971224 0.81007) (xy -0.829855 0.822844)
    (xy -0.738793 0.841504) (xy -0.684052 0.86705) (xy -0.668022 0.880574) (xy -0.591513 1.013014) (xy -0.612942 1.169326)
    (xy -0.639527 1.225669) (xy -0.661032 1.256613) (xy -0.696666 1.280644) (xy -0.758809 1.298631) (xy -0.859839 1.311446)
    (xy -1.012135 1.31996) (xy -1.228075 1.325042) (xy -1.520037 1.327564) (xy -1.900401 1.328397) (xy -2.100824 1.328452)
    (xy -3.507113 1.328452) (xy -3.507113 -4.782427) (xy -5.885042 -4.781907) (xy -8.262971 -4.781388) (xy -8.528661 -4.657114)
    (xy -8.718832 -4.543626) (xy -8.916181 -4.3885) (xy -9.016631 -4.290713) (xy -9.106619 -4.18959) (xy -9.181539 -4.092709)
    (xy -9.24277 -3.989611) (xy -9.291691 -3.869836) (xy -9.329682 -3.722926) (xy -9.358121 -3.538422) (xy -9.378388 -3.305864)
    (xy -9.391863 -3.014793) (xy -9.399923 -2.65475) (xy -9.403948 -2.215277) (xy -9.405318 -1.685914) (xy -9.40544 -1.34211)
    (xy -9.40544 0.803603) (xy -9.966955 0.803603) (xy -9.97851 -0.983054) (xy -9.981361 -1.670357) (xy -9.980438 -2.262126)
    (xy -9.975774 -2.756334) (xy -9.967401 -3.150954) (xy -9.955354 -3.443957) (xy -9.939664 -3.633317) (xy -9.934834 -3.66626)
    (xy -9.806832 -4.11648) (xy -9.587721 -4.51489) (xy -9.282662 -4.854698) (xy -8.896816 -5.129111) (xy -8.77422 -5.193688)
    (xy -8.475523 -5.340376) (xy -5.699059 -5.355466) (xy -2.922594 -5.370555))
   (layer "F.Cu") (width 0) (fill solid)))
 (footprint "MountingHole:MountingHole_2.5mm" (layer "F.Cu") (at 192 72 180)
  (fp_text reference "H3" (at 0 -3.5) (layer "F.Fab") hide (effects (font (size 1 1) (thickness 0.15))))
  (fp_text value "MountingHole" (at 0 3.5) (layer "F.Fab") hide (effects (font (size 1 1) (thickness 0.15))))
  (pad "" np_thru_hole circle (at 0 0 180) (size 2.5 2.5) (drill 2.5) (layers *.Cu *.Mask)))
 (gr_line (start 115 72) (end 115 123) (layer "Edge.Cuts") (width 0.1))
 (gr_line (start 174.5 124) (end 174.5 118.5) (layer "Edge.Cuts") (width 0.1))
 (gr_arc (start 174.5 124) (mid 173.62132 126.12132) (end 171.5 127) (layer "Edge.Cuts") (width 0.1))
 (gr_line (start 119 127) (end 171.5 127) (layer "Edge.Cuts") (width 0.1))
 (gr_line (start 193 115.5) (end 177.5 115.5) (layer "Edge.Cuts") (width 0.1))
 (gr_arc (start 119 127) (mid 116.171573 125.828427) (end 115 123) (layer "Edge.Cuts") (width 0.1))
 (gr_arc (start 115 72) (mid 116.171573 69.171573) (end 119 68) (layer "Edge.Cuts") (width 0.1))
 (gr_arc (start 174.5 118.5) (mid 175.37868 116.37868) (end 177.5 115.5) (layer "Edge.Cuts") (width 0.1))
 (gr_line (start 196 112.5) (end 196 72) (layer "Edge.Cuts") (width 0.1))
 (gr_line (start 192 68) (end 119 68) (layer "Edge.Cuts") (width 0.1))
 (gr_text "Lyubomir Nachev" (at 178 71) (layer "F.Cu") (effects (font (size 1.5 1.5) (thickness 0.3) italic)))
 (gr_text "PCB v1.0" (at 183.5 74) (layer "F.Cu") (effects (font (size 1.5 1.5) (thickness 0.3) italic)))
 (segment (start 176.88 82.38) (end 173.8 79.3) (width 0.5) (layer "F.Cu") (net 14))
 (segment (start 181.5 87) (end 181.5 109.5) (width 0.5) (layer "F.Cu") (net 14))
 (segment (start 169.93 94.54) (end 152.46 94.54) (width 0.5) (layer "F.Cu") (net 14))
 (segment (start 139.81 94.69) (end 141 94.69) (width 0.5) (layer "F.Cu") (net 14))
 (segment (start 150.5 110.5) (end 148.72 112.28) (width 0.5) (layer "F.Cu") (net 14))
 (segment (start 169.93 94.54) (end 171.96 94.54) (width 0.5) (layer "F.Cu") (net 14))
 (segment (start 178.195 85.695) (end 179.5 87) (width 0.5) (layer "F.Cu") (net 14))
 (segment (start 180 111) (end 175.5 111) (width 0.5) (layer "F.Cu") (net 14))
 (segment (start 173.5 93) (end 173.5 87) (width 0.5) (layer "F.Cu") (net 14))
 (segment (start 140.78 112.28) (end 139 110.5) (width 0.5) (layer "F.Cu") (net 14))
 (segment (start 174.5 104) (end 175.025 103.475) (width 0.5) (layer "F.Cu") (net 14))
 (segment (start 179.5 87) (end 179.5 102.5) (width 0.5) (layer "F.Cu") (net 14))
 (segment (start 176.88 85.695) (end 178.195 85.695) (width 0.5) (layer "F.Cu") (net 14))
 (segment (start 139 95.5) (end 139.81 94.69) (width 0.5) (layer "F.Cu") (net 14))
 (segment (start 176.88 82.38) (end 176.88 85.695) (width 0.5) (layer "F.Cu") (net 14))
 (segment (start 147.07 112.28) (end 140.78 112.28) (width 0.5) (layer "F.Cu") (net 14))
 (segment (start 148.72 112.28) (end 147.07 112.28) (width 0.5) (layer "F.Cu") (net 14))
 (segment (start 174.5 110) (end 174.5 104) (width 0.5) (layer "F.Cu") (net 14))
 (segment (start 192.12 85.695) (end 182.805 85.695) (width 0.5) (layer "F.Cu") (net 14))
 (segment (start 174.805 85.695) (end 176.88 85.695) (width 0.5) (layer "F.Cu") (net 14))
 (segment (start 179.5 102.5) (end 178.525 103.475) (width 0.5) (layer "F.Cu") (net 14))
 (segment (start 150.5 96.5) (end 150.5 110.5) (width 0.5) (layer "F.Cu") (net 14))
 (segment (start 171.96 94.54) (end 173.5 93) (width 0.5) (layer "F.Cu") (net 14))
 (segment (start 175.025 103.475) (end 176.88 103.475) (width 0.5) (layer "F.Cu") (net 14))
 (segment (start 173.5 87) (end 174.805 85.695) (width 0.5) (layer "F.Cu") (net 14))
 (segment (start 182.805 85.695) (end 181.5 87) (width 0.5) (layer "F.Cu") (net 14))
 (segment (start 152.46 94.54) (end 150.5 96.5) (width 0.5) (layer "F.Cu") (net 14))
 (segment (start 175.5 111) (end 174.5 110) (width 0.5) (layer "F.Cu") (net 14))
 (segment (start 181.5 109.5) (end 180 111) (width 0.5) (layer "F.Cu") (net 14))
 (segment (start 139 110.5) (end 139 95.5) (width 0.5) (layer "F.Cu") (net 14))
 (segment (start 173.8 79.3) (end 169.93 79.3) (width 0.5) (layer "F.Cu") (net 14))
 (segment (start 178.525 103.475) (end 176.88 103.475) (width 0.5) (layer "F.Cu") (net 14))
 (segment (start 147.07 79.26) (end 144.74 79.26) (width 0.5) (layer "F.Cu") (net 1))
 (segment (start 178.985 106.015) (end 176.88 106.015) (width 0.5) (layer "F.Cu") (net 1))
 (segment (start 142.27 97.23) (end 141 97.23) (width 0.5) (layer "F.Cu") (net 1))
 (segment (start 178.5 76) (end 180.5 78) (width 0.5) (layer "F.Cu") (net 1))
 (segment (start 180.5 104.5) (end 178.985 106.015) (width 0.5) (layer "F.Cu") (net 1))
 (segment (start 147.07 76.93) (end 148 76) (width 0.5) (layer "F.Cu") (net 1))
 (segment (start 180.5 78) (end 180.5 104.5) (width 0.5) (layer "F.Cu") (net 1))
 (segment (start 144.74 79.26) (end 143 81) (width 0.5) (layer "F.Cu") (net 1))
 (segment (start 148 76) (end 178.5 76) (width 0.5) (layer "F.Cu") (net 1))
 (segment (start 143 96.5) (end 142.27 97.23) (width 0.5) (layer "F.Cu") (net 1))
 (segment (start 143 81) (end 143 96.5) (width 0.5) (layer "F.Cu") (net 1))
 (segment (start 147.07 79.26) (end 147.07 76.93) (width 0.5) (layer "F.Cu") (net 1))
 (segment (start 145 101.5) (end 144.19 102.31) (width 0.5) (layer "F.Cu") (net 6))
 (segment (start 144.19 102.31) (end 141 102.31) (width 0.5) (layer "F.Cu") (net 6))
 (segment (start 147.07 91.96) (end 145.54 91.96) (width 0.5) (layer "F.Cu") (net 6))
 (segment (start 145 92.5) (end 145 101.5) (width 0.5) (layer "F.Cu") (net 6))
 (segment (start 145.54 91.96) (end 145 92.5) (width 0.5) (layer "F.Cu") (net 6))
 (segment (start 147.07 89.42) (end 145.08 89.42) (width 0.5) (layer "F.Cu") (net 5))
 (segment (start 144 90.5) (end 144 99) (width 0.5) (layer "F.Cu") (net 5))
 (segment (start 144 99) (end 143.23 99.77) (width 0.5) (layer "F.Cu") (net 5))
 (segment (start 141 99.77) (end 143.23 99.77) (width 0.5) (layer "F.Cu") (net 5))
 (segment (start 145.08 89.42) (end 144 90.5) (width 0.5) (layer "F.Cu") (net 5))
 (segment (start 169.93 102.16) (end 171.84 102.16) (width 0.5) (layer "F.Cu") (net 27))
 (segment (start 172.5 99) (end 173.105 98.395) (width 0.5) (layer "F.Cu") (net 27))
 (segment (start 171.84 102.16) (end 172.5 101.5) (width 0.5) (layer "F.Cu") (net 27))
 (segment (start 172.5 101.5) (end 172.5 99) (width 0.5) (layer "F.Cu") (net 27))
 (segment (start 173.105 98.395) (end 176.88 98.395) (width 0.5) (layer "F.Cu") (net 27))
 (segment (start 176.88 100.935) (end 174.565 100.935) (width 0.5) (layer "F.Cu") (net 30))
 (segment (start 173.5 102) (end 173.5 108.5) (width 0.5) (layer "F.Cu") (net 30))
 (segment (start 174.565 100.935) (end 173.5 102) (width 0.5) (layer "F.Cu") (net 30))
 (segment (start 172.22 109.78) (end 169.93 109.78) (width 0.5) (layer "F.Cu") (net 30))
 (segment (start 173.5 108.5) (end 172.22 109.78) (width 0.5) (layer "F.Cu") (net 30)))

